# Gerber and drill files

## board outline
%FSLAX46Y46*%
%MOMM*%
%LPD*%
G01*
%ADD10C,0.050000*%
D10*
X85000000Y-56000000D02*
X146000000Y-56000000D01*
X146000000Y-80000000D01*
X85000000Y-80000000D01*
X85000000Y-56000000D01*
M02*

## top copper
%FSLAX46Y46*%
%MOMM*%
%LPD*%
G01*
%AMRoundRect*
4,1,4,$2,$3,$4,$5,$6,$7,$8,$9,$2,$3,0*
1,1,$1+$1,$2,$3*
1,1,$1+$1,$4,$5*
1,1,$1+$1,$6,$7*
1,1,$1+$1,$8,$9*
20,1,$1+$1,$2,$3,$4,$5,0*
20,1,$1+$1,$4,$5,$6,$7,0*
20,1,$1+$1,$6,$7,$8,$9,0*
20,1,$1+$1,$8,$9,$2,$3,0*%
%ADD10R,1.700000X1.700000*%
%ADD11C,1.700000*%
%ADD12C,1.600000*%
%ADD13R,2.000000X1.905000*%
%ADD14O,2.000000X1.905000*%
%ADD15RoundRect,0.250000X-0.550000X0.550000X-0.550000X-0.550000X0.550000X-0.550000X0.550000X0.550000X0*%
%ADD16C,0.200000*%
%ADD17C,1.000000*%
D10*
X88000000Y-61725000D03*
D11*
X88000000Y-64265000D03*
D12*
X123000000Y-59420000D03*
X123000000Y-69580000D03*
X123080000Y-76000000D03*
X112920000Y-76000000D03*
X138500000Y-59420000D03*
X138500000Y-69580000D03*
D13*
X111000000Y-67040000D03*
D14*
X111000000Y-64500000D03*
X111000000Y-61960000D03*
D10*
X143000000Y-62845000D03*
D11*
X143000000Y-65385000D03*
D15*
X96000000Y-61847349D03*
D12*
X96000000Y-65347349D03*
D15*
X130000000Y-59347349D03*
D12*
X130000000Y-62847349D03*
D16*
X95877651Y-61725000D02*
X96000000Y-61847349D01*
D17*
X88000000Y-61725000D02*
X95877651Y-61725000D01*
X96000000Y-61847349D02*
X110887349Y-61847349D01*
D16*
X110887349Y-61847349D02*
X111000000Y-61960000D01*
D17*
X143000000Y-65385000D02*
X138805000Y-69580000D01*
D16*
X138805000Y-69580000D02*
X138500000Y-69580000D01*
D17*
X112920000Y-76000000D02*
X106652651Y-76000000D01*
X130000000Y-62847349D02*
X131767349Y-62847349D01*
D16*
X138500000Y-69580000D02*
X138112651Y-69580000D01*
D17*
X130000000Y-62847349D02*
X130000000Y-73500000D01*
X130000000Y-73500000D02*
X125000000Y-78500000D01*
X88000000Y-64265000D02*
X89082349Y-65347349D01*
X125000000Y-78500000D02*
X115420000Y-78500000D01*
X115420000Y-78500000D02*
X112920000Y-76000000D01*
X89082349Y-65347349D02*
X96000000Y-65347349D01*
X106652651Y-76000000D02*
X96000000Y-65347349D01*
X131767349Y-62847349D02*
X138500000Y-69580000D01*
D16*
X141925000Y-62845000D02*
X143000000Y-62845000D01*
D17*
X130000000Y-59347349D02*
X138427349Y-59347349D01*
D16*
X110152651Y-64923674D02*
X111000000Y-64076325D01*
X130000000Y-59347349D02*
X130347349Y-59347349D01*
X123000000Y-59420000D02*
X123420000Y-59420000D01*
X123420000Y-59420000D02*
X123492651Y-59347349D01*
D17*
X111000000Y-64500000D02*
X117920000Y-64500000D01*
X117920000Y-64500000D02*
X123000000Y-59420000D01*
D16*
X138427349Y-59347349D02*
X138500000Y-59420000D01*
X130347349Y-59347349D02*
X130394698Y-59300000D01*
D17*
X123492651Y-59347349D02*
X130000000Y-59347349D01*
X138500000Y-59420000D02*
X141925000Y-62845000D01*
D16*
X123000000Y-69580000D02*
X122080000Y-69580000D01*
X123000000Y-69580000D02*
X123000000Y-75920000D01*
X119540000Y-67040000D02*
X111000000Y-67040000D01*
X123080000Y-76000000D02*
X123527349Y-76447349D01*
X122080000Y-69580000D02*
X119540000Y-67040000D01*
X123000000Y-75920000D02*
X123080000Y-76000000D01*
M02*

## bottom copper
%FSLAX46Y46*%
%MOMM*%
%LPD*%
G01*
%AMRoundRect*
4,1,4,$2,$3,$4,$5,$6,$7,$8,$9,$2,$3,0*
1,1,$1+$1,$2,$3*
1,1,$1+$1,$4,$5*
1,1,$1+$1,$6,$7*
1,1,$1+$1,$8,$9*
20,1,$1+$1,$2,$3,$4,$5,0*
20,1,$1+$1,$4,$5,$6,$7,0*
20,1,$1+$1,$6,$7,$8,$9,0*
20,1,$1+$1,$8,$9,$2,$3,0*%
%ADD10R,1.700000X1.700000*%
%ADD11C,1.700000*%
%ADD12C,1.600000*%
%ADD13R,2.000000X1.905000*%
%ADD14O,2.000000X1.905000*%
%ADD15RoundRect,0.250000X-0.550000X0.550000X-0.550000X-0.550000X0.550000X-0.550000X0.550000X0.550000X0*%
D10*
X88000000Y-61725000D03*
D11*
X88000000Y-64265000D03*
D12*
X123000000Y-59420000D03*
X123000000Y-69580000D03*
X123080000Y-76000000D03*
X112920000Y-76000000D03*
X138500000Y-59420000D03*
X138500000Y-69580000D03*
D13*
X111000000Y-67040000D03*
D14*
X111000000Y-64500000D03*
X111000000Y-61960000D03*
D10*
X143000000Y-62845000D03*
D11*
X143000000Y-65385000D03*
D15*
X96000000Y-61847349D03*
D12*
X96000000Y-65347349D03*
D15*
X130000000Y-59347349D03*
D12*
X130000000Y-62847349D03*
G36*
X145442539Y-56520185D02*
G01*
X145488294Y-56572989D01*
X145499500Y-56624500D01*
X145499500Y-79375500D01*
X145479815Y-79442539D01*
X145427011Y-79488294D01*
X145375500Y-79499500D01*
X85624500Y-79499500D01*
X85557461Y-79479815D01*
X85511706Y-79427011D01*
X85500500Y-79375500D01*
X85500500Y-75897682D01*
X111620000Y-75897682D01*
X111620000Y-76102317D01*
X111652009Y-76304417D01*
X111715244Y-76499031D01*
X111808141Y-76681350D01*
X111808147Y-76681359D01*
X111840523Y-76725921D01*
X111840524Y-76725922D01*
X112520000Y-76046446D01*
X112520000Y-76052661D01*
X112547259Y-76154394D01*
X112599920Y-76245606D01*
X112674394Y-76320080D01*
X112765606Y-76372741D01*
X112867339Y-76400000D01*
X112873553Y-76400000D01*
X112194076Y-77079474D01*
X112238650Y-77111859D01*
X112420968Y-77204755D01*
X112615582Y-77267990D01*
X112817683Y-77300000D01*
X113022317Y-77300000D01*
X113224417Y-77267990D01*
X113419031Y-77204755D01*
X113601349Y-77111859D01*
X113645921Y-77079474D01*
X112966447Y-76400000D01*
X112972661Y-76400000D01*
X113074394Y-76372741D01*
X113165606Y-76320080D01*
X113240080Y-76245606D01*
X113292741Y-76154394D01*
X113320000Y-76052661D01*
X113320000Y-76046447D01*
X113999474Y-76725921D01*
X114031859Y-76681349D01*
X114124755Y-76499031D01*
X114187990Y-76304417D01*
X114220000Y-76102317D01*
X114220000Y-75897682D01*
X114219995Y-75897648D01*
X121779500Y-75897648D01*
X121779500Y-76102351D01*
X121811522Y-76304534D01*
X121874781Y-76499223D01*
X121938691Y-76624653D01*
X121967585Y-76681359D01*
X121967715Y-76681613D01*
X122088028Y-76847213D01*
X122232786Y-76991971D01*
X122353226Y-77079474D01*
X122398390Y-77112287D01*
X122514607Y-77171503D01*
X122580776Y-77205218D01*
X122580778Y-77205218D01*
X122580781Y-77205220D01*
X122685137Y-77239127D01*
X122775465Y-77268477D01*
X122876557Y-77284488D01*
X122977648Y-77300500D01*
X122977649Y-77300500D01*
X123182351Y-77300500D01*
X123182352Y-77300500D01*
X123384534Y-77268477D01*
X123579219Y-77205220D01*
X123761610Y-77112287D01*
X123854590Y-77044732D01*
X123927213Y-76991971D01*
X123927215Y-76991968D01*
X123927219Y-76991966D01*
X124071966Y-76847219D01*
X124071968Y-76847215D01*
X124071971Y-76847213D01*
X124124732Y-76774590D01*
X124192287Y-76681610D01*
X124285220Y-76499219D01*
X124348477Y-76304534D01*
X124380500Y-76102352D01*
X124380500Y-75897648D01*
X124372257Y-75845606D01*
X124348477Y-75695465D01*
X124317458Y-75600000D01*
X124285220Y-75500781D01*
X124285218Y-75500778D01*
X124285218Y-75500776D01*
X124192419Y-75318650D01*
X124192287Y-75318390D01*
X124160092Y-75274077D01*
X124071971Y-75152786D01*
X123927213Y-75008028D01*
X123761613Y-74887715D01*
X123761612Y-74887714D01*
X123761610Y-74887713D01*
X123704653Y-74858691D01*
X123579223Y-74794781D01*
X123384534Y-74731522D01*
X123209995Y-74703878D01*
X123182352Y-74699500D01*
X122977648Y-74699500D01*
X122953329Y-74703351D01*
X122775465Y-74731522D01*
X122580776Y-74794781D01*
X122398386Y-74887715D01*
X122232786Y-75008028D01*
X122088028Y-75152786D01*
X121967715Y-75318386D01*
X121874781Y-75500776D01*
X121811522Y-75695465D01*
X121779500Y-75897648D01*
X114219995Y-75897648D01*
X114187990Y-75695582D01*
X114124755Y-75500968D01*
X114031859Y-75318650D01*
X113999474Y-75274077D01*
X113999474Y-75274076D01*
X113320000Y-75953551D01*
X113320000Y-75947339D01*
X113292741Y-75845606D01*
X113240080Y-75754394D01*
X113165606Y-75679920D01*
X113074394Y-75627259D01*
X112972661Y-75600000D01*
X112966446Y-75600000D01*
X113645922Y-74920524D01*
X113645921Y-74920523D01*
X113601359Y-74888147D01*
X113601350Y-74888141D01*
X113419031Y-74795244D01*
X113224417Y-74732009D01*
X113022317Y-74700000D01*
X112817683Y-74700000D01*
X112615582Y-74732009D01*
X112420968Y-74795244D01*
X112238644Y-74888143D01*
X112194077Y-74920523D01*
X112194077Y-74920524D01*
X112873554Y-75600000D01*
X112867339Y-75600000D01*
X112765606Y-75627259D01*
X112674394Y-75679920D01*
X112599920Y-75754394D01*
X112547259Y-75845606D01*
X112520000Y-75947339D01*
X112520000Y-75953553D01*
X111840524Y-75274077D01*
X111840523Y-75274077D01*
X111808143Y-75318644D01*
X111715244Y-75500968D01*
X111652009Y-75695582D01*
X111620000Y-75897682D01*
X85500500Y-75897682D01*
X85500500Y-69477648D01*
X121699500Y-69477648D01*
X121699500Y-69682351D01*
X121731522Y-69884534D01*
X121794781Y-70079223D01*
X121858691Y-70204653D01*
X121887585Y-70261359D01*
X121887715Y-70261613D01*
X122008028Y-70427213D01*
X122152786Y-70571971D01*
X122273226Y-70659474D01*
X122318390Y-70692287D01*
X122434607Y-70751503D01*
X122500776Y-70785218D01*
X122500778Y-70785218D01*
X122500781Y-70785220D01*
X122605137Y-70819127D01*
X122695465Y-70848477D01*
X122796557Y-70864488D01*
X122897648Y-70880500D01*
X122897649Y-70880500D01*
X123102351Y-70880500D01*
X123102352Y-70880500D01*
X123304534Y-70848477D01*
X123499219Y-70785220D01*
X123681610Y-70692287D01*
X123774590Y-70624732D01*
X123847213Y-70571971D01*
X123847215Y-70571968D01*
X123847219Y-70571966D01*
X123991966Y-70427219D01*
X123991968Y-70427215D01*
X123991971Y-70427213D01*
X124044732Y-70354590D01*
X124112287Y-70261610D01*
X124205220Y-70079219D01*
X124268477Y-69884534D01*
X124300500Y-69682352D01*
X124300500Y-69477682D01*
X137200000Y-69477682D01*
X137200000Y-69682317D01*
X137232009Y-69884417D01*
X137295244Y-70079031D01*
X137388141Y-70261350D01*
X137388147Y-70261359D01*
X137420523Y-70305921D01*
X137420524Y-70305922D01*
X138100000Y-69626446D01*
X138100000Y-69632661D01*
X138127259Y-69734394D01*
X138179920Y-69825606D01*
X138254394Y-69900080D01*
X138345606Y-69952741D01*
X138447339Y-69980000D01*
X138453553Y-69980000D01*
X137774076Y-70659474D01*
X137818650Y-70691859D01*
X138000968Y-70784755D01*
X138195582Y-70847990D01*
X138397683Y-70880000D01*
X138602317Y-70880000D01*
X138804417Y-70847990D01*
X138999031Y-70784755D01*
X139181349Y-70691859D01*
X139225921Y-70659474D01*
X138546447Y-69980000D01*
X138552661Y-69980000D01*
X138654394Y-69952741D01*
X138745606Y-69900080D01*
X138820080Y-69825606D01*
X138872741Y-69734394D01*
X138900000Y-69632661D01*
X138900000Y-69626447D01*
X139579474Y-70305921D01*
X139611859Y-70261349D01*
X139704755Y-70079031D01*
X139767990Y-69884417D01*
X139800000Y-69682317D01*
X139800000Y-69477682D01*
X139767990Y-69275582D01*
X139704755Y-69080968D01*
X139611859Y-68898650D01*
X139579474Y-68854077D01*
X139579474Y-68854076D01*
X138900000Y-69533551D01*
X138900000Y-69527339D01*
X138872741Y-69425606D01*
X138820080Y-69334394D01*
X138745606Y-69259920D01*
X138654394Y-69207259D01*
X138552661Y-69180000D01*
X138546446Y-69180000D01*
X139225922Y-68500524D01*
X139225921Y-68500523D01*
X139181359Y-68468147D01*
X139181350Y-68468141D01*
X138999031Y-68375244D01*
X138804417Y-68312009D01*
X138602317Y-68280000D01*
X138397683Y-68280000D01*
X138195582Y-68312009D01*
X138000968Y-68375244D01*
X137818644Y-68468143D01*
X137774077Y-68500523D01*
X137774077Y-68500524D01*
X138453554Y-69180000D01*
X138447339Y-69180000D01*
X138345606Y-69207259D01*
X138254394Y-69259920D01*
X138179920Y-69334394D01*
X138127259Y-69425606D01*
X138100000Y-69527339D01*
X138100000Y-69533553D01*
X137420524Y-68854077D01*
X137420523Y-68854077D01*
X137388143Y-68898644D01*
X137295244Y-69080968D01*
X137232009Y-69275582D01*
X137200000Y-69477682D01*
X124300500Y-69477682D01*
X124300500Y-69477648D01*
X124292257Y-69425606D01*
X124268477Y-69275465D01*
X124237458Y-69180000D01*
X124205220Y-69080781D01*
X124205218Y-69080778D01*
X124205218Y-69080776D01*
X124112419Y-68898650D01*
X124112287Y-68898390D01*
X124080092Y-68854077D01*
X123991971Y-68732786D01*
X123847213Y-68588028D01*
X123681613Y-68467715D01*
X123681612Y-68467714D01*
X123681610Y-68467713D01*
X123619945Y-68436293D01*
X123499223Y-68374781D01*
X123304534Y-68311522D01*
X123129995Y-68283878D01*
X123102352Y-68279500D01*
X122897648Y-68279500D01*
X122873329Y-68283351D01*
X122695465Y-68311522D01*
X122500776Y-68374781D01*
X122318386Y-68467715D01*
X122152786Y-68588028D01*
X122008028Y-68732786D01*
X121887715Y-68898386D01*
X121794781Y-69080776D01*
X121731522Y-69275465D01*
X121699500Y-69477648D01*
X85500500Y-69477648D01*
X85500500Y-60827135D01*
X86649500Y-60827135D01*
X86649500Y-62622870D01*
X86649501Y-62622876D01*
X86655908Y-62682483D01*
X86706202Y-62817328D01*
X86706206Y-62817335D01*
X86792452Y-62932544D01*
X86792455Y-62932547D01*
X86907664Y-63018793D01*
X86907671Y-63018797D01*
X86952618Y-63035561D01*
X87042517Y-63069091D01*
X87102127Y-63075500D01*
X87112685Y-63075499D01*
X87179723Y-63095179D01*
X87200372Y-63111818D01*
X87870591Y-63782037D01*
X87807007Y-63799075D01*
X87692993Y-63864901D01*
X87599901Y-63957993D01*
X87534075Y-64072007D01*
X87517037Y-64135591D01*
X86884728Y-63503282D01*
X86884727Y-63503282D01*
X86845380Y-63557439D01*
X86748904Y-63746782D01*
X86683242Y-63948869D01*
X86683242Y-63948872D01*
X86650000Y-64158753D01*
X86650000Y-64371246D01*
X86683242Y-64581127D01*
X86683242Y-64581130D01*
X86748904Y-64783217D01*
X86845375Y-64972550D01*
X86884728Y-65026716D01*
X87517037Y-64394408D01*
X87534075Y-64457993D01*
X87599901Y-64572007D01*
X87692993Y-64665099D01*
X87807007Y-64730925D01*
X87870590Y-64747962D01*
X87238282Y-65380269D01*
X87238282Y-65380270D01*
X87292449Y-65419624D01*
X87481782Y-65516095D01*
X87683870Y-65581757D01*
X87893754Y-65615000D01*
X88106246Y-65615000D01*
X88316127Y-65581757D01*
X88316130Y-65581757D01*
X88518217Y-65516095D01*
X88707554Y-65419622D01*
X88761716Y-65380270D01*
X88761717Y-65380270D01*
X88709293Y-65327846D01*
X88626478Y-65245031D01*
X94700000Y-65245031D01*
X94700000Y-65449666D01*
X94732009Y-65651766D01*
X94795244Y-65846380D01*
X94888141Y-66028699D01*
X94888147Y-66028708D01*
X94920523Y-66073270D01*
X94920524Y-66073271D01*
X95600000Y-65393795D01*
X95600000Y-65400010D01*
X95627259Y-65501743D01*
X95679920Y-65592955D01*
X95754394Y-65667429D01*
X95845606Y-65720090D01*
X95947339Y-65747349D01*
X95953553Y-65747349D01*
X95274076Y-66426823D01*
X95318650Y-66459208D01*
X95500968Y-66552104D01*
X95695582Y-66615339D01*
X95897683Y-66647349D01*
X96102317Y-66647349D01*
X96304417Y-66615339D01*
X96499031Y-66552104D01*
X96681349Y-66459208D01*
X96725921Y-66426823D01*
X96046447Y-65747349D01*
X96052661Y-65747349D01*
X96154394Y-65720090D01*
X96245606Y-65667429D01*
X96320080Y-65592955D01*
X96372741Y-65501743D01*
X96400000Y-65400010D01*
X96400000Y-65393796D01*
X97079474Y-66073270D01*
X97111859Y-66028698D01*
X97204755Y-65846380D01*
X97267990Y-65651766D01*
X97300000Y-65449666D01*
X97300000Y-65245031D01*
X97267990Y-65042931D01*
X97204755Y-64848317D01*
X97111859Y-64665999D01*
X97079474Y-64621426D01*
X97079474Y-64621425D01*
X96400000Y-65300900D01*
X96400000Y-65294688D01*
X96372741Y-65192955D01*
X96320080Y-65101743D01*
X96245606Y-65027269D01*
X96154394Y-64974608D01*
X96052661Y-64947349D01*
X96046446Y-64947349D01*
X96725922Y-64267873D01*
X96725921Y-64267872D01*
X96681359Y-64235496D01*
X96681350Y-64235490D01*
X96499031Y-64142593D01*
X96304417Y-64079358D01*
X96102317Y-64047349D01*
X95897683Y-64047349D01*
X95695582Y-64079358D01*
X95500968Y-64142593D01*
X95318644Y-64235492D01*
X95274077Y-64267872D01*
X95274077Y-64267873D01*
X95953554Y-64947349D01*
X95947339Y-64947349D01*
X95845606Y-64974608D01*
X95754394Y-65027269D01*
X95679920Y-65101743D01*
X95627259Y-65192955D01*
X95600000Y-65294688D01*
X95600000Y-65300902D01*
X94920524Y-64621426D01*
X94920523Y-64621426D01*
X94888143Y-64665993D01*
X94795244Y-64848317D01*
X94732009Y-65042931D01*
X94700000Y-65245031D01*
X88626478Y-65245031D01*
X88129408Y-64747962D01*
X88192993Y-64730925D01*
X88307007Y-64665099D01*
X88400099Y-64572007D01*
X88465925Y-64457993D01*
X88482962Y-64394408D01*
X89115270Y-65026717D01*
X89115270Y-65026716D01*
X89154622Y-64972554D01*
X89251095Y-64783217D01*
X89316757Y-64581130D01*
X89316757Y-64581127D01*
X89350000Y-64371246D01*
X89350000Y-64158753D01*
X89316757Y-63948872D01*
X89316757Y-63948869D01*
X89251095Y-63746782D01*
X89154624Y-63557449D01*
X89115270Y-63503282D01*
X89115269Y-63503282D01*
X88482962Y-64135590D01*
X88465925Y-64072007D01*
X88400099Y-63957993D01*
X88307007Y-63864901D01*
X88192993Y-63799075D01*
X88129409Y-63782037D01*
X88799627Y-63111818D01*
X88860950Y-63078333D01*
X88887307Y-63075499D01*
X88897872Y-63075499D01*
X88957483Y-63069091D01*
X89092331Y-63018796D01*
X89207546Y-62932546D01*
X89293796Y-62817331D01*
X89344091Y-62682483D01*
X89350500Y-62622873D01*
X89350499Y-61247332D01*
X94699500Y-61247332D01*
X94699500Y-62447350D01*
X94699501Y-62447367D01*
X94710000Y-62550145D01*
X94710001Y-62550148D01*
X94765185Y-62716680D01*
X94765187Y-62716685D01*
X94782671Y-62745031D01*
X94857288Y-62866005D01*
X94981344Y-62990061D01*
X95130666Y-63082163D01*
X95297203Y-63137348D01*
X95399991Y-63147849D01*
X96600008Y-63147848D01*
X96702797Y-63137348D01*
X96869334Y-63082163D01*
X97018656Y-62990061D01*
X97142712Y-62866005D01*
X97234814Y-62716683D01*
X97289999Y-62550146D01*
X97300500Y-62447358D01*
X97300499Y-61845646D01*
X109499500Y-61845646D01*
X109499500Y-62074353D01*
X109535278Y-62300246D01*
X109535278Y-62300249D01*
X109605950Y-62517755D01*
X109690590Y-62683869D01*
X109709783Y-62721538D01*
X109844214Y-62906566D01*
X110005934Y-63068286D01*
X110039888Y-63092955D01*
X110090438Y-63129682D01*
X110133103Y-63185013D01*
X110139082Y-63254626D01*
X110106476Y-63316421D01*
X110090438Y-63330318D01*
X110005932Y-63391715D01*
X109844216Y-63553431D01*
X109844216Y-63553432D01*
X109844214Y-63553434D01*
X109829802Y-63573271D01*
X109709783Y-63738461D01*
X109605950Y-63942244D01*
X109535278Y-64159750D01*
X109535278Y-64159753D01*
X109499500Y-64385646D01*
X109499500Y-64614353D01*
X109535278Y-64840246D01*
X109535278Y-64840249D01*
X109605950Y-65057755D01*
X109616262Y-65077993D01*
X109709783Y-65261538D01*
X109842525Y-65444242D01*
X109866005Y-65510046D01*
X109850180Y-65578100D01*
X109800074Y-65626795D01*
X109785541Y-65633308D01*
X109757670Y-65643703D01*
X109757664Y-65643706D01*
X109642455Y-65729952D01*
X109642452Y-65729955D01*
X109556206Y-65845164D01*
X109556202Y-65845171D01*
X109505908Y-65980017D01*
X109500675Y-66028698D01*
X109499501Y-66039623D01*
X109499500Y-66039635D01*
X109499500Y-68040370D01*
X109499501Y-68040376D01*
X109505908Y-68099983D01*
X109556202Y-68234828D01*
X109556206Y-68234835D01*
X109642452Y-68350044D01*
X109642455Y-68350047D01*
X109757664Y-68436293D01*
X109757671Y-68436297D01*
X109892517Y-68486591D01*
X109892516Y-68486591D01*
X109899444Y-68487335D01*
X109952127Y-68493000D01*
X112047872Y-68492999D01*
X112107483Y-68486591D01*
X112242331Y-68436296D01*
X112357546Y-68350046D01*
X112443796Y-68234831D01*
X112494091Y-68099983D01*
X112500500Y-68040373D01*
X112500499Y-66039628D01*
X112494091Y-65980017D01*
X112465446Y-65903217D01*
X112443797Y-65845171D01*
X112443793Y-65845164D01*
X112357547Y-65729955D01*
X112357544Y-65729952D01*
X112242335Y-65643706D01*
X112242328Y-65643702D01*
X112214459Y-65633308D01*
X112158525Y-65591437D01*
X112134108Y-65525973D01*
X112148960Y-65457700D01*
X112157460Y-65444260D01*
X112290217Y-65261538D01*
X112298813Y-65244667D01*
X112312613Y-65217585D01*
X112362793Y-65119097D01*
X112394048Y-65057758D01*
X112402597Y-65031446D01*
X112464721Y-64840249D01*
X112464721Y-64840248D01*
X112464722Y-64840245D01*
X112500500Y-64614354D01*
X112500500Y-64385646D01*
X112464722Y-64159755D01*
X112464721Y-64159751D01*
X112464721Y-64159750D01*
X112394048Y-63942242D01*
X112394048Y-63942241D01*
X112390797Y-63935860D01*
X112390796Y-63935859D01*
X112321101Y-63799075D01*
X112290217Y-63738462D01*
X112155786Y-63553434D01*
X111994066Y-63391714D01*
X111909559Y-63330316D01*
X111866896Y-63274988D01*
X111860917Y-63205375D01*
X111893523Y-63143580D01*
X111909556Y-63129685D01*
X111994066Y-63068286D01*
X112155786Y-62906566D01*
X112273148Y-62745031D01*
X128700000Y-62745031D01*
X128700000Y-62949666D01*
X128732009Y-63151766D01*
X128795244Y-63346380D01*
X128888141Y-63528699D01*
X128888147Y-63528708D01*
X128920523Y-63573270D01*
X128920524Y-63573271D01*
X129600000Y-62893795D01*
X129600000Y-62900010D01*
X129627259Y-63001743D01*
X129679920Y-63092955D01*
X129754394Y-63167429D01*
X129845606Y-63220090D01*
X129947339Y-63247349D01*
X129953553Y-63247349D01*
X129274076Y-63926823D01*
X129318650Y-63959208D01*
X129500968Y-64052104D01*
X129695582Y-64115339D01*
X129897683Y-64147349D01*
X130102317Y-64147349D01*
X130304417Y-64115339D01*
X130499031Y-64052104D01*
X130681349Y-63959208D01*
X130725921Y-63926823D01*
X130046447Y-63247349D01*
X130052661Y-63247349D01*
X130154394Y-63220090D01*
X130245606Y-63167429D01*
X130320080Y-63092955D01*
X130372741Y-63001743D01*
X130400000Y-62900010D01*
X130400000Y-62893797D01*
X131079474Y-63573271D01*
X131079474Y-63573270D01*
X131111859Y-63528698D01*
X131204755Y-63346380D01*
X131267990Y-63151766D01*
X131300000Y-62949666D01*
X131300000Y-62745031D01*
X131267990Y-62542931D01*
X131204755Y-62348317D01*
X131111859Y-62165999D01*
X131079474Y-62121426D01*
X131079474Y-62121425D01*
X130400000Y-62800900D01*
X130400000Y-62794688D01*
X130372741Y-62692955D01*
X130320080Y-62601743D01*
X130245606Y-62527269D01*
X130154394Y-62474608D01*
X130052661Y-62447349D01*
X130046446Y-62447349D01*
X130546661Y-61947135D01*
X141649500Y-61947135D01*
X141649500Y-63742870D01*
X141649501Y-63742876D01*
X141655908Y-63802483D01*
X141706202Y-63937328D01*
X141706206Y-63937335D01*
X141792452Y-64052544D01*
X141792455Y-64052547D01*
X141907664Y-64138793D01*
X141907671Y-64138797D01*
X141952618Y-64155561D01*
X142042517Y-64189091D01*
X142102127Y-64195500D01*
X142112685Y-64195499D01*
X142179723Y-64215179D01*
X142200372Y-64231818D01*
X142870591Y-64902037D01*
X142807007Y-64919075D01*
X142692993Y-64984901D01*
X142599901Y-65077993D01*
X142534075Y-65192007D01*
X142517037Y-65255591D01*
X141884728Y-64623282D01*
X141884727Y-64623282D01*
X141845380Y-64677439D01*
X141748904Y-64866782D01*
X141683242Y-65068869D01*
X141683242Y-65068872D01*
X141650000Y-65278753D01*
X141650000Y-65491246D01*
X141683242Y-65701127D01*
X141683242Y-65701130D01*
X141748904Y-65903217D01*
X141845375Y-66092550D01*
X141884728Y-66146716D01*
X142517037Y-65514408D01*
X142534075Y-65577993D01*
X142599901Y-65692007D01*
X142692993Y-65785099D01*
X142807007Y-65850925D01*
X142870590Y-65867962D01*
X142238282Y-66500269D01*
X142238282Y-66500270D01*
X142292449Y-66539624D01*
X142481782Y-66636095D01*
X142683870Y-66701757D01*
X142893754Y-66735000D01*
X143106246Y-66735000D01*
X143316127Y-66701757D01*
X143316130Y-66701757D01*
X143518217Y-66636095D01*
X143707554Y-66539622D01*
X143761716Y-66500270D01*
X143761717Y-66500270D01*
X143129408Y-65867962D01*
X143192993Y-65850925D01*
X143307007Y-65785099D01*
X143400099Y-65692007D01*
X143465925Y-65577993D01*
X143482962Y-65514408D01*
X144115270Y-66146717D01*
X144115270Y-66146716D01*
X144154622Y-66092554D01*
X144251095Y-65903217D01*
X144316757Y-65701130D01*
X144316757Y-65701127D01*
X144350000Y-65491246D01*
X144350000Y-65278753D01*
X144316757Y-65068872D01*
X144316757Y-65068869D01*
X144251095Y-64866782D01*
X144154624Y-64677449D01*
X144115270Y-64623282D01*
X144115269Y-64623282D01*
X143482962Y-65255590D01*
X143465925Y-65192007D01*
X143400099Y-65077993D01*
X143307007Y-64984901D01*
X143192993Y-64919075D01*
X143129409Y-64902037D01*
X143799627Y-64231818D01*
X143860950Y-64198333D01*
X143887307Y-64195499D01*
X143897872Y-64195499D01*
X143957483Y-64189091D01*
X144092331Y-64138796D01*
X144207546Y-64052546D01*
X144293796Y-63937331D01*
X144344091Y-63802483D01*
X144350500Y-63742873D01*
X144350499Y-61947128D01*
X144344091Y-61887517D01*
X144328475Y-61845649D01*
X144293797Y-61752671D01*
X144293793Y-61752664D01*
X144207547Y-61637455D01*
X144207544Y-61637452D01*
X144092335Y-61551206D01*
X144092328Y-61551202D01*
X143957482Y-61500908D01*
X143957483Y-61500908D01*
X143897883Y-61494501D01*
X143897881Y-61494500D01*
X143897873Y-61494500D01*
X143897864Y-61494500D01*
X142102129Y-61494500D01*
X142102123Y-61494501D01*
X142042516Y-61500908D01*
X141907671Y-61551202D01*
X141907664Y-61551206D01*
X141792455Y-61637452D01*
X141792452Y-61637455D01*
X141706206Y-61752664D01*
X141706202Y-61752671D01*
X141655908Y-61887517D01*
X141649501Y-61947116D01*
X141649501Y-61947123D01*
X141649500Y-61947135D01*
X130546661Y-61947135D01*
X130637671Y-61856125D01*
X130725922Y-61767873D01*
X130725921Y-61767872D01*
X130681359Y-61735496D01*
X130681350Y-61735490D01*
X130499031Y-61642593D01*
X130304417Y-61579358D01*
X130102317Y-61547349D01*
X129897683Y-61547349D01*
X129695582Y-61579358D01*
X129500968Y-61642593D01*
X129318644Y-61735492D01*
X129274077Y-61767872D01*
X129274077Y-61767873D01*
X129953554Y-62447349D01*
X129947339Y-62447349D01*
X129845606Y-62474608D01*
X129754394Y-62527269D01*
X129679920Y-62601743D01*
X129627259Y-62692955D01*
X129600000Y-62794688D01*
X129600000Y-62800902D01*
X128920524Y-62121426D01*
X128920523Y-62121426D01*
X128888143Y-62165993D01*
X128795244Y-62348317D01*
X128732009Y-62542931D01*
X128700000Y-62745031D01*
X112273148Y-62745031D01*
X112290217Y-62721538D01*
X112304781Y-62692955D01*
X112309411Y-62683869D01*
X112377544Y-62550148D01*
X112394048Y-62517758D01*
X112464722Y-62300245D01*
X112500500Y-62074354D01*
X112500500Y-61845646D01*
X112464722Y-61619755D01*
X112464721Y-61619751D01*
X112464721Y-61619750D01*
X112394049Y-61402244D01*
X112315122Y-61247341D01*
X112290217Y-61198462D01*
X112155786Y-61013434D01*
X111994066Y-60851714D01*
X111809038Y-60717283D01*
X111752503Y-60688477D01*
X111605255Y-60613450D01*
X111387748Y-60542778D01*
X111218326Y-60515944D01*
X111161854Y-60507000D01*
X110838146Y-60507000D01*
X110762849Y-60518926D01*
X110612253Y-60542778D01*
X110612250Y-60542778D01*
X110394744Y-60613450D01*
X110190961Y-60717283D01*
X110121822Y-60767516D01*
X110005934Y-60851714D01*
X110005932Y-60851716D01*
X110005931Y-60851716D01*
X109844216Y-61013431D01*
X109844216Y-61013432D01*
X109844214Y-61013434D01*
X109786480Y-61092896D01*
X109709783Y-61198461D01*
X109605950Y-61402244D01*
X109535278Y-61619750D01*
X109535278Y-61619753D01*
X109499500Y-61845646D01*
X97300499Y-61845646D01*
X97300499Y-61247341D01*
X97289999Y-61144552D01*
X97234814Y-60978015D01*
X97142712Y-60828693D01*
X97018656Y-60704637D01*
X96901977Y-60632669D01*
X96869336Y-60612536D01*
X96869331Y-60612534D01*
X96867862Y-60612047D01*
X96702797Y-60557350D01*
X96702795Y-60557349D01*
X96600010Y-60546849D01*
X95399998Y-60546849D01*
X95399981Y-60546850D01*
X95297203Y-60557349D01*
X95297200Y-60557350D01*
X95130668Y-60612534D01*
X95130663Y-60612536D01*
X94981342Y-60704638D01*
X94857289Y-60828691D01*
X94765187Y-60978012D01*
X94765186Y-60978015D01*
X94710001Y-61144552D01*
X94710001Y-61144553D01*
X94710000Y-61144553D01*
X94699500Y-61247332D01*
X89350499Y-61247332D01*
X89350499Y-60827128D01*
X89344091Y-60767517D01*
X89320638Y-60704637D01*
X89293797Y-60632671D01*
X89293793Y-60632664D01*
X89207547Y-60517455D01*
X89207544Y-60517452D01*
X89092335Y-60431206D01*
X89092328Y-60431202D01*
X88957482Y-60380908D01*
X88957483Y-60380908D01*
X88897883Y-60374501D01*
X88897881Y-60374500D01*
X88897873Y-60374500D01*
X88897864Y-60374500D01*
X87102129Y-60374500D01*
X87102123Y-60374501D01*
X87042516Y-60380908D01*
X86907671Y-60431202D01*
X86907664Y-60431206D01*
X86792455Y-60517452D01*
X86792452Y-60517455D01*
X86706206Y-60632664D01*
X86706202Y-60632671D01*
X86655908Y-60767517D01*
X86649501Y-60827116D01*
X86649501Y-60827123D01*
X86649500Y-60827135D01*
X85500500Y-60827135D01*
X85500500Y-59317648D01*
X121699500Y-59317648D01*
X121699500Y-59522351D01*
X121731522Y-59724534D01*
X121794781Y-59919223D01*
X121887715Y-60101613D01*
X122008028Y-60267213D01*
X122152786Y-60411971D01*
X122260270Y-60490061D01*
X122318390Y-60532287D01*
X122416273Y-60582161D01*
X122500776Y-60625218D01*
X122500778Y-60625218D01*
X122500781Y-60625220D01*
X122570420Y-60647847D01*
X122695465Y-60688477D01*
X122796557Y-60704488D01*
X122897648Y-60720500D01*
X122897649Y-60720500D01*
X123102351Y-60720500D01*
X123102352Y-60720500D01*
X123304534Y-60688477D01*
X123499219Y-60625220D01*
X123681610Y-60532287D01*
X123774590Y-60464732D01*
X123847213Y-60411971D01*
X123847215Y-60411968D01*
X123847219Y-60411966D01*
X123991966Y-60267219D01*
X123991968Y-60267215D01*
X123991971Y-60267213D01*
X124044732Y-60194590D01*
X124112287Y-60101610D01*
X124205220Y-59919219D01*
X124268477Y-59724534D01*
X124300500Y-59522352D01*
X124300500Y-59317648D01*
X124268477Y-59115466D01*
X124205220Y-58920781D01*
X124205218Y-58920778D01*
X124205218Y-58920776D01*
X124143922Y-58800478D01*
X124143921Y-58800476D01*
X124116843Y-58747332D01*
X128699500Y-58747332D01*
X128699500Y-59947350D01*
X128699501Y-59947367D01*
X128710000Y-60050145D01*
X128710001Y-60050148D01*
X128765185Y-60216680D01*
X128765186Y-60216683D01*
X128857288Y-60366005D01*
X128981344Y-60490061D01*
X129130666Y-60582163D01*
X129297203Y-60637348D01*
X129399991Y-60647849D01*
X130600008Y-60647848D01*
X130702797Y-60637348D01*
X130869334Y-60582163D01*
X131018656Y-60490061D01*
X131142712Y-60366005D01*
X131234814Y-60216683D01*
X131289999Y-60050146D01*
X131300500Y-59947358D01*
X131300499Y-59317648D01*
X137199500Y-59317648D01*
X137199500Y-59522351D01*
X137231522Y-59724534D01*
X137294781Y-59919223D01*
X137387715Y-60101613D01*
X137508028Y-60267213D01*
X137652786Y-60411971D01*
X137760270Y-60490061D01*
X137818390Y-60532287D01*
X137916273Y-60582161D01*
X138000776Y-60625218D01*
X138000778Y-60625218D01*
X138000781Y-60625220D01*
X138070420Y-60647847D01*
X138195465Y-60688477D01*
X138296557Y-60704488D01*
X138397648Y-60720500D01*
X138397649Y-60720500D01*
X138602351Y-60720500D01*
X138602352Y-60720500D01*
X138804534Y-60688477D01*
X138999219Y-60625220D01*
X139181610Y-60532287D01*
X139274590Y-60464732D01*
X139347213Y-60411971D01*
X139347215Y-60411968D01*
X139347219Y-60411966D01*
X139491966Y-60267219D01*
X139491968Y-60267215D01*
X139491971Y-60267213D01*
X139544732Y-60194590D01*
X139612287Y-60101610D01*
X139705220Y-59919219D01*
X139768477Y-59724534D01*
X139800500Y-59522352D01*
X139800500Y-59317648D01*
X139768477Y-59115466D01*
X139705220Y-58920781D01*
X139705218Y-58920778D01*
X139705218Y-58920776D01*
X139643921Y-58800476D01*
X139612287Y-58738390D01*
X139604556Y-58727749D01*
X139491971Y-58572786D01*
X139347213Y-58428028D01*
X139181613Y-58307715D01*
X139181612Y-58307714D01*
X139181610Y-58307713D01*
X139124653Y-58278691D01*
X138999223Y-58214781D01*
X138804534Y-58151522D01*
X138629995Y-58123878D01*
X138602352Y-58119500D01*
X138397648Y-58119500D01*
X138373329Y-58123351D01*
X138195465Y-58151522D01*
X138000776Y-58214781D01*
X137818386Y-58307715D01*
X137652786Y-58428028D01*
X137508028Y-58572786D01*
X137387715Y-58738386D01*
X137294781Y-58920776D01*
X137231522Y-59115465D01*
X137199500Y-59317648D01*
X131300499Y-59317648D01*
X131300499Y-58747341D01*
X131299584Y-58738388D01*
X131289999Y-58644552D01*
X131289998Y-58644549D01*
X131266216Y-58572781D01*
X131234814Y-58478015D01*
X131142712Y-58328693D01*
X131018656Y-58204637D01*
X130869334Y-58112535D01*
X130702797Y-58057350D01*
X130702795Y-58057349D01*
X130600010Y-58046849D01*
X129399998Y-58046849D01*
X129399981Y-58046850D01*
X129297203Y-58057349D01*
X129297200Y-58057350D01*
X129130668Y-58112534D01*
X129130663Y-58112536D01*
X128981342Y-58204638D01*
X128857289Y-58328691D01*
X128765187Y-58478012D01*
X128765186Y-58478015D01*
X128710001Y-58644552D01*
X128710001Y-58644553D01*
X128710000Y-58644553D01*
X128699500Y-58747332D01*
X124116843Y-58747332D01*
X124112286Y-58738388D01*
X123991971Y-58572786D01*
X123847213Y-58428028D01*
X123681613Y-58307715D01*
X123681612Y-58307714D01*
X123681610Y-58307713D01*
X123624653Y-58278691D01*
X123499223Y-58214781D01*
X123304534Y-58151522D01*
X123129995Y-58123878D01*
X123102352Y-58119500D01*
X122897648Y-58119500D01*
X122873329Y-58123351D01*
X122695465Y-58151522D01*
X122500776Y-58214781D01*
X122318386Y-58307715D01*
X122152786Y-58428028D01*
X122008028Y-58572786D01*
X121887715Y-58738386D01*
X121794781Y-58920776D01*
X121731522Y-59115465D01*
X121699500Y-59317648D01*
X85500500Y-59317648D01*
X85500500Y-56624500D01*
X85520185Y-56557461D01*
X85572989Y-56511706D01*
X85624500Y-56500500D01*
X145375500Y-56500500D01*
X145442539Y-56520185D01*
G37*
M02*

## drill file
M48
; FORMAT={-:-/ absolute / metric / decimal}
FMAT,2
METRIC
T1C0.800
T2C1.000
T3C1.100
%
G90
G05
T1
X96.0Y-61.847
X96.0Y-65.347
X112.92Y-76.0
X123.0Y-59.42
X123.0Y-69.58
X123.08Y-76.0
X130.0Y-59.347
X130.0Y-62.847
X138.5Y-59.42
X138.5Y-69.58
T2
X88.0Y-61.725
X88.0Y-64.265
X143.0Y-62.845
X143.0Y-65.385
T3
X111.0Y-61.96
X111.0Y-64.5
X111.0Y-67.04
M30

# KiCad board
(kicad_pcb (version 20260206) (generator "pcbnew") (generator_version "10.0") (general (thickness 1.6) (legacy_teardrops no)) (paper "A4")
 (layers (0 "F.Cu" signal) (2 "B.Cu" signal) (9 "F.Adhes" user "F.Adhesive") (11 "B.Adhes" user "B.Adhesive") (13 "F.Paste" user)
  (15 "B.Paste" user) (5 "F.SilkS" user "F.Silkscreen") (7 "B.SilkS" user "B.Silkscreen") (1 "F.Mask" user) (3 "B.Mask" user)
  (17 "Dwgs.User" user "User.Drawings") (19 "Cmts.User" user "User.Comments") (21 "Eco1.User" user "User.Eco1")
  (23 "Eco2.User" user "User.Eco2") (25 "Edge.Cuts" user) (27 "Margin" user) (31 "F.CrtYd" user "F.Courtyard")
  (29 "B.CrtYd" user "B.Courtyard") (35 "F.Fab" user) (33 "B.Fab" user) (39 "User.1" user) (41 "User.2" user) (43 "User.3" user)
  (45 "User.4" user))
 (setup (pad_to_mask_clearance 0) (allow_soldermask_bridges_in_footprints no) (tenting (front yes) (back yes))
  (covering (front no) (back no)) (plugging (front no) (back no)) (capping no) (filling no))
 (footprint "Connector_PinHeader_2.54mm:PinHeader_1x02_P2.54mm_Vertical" (layer "F.Cu") (at 88 61.725)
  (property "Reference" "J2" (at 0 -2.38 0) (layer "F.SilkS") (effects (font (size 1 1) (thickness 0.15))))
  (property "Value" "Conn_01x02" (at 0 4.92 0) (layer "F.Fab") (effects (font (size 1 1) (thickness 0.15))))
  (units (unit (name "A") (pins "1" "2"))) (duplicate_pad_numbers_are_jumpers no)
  (pad "1" thru_hole rect (at 0 0) (size 1.7 1.7) (drill 1) (layers "*.Cu" "*.Mask") (remove_unused_layers no) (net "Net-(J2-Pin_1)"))
  (pad "2" thru_hole circle (at 0 2.54) (size 1.7 1.7) (drill 1) (layers "*.Cu" "*.Mask") (remove_unused_layers no) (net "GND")))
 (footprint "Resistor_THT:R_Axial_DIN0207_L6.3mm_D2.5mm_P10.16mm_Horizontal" (layer "F.Cu") (at 123 59.42 -90)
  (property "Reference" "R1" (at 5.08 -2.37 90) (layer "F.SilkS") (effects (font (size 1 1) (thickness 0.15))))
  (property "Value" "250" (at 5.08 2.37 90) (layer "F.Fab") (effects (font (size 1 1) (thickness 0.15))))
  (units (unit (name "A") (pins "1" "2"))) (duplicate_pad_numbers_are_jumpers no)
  (pad "1" thru_hole circle (at 0 0 270) (size 1.6 1.6) (drill 0.8) (layers "*.Cu" "*.Mask") (remove_unused_layers no)
   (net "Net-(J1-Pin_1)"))
  (pad "2" thru_hole circle (at 10.16 0 270) (size 1.6 1.6) (drill 0.8) (layers "*.Cu" "*.Mask") (remove_unused_layers no)
   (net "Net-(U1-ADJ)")))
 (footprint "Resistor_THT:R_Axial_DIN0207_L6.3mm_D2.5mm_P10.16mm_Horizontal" (layer "F.Cu") (at 123.08 76 180)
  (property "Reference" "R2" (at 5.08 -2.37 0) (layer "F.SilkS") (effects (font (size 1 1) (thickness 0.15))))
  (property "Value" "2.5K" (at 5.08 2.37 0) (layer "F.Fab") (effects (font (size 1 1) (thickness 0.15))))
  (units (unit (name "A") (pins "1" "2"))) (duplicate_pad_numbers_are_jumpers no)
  (pad "1" thru_hole circle (at 0 0 180) (size 1.6 1.6) (drill 0.8) (layers "*.Cu" "*.Mask") (remove_unused_layers no) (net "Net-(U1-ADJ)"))
  (pad "2" thru_hole circle (at 10.16 0 180) (size 1.6 1.6) (drill 0.8) (layers "*.Cu" "*.Mask") (remove_unused_layers no) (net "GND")))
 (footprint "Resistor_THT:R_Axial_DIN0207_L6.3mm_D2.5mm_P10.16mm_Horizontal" (layer "F.Cu") (at 138.5 59.42 -90)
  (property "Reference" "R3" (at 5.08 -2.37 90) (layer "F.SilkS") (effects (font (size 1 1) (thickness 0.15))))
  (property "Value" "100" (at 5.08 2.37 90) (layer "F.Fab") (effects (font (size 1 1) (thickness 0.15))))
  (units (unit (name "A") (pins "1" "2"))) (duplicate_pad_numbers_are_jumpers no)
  (pad "1" thru_hole circle (at 0 0 270) (size 1.6 1.6) (drill 0.8) (layers "*.Cu" "*.Mask") (remove_unused_layers no)
   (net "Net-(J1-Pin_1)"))
  (pad "2" thru_hole circle (at 10.16 0 270) (size 1.6 1.6) (drill 0.8) (layers "*.Cu" "*.Mask") (remove_unused_layers no) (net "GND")))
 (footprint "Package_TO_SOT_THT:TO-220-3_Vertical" (layer "F.Cu") (at 111 67.04 90)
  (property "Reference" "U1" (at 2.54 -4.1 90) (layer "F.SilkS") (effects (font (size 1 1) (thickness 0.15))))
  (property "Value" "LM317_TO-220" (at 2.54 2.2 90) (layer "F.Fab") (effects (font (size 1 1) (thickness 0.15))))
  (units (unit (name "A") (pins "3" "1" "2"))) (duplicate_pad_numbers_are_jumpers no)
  (pad "1" thru_hole rect (at 0 0 90) (size 1.905 2) (drill 1.1) (layers "*.Cu" "*.Mask") (remove_unused_layers no) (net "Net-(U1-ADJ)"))
  (pad "2" thru_hole oval (at 2.54 0 90) (size 1.905 2) (drill 1.1) (layers "*.Cu" "*.Mask") (remove_unused_layers no)
   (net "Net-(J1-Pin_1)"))
  (pad "3" thru_hole oval (at 5.08 0 90) (size 1.905 2) (drill 1.1) (layers "*.Cu" "*.Mask") (remove_unused_layers no)
   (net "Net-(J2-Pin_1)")))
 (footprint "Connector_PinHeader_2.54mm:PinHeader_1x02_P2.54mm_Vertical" (layer "F.Cu") (at 143 62.845)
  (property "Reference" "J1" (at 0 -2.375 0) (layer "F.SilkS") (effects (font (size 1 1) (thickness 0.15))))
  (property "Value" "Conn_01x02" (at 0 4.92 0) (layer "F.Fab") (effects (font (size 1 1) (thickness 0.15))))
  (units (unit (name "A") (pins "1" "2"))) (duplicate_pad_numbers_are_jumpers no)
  (pad "1" thru_hole rect (at 0 0) (size 1.7 1.7) (drill 1) (layers "*.Cu" "*.Mask") (remove_unused_layers no) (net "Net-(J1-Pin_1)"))
  (pad "2" thru_hole circle (at 0 2.54) (size 1.7 1.7) (drill 1) (layers "*.Cu" "*.Mask") (remove_unused_layers no) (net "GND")))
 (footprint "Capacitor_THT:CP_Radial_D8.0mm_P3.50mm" (layer "F.Cu") (at 96 61.847349 -90)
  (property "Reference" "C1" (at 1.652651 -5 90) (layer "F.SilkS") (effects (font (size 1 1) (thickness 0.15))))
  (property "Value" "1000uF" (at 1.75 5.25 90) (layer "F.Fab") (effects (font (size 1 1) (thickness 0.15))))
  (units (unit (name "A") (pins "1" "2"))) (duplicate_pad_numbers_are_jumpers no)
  (pad "1" thru_hole roundrect (at 0 0 270) (size 1.6 1.6) (drill 0.8) (layers "*.Cu" "*.Mask") (remove_unused_layers no)
   (roundrect_rratio 0.15625) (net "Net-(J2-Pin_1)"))
  (pad "2" thru_hole circle (at 3.5 0 270) (size 1.6 1.6) (drill 0.8) (layers "*.Cu" "*.Mask") (remove_unused_layers no) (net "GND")))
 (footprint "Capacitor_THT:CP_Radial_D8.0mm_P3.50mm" (layer "F.Cu") (at 130 59.347349 -90)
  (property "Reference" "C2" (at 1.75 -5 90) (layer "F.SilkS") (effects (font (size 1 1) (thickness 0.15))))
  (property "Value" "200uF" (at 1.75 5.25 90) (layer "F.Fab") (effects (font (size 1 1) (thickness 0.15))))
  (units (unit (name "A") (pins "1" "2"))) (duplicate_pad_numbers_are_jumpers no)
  (pad "1" thru_hole roundrect (at 0 0 270) (size 1.6 1.6) (drill 0.8) (layers "*.Cu" "*.Mask") (remove_unused_layers no)
   (roundrect_rratio 0.15625) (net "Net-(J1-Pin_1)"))
  (pad "2" thru_hole circle (at 3.5 0 270) (size 1.6 1.6) (drill 0.8) (layers "*.Cu" "*.Mask") (remove_unused_layers no) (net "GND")))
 (gr_rect (start 85 56) (end 146 80) (stroke (width 0.05) (type default)) (fill no) (layer "Edge.Cuts"))
 (segment (start 95.877651 61.725) (end 96 61.847349) (width 0.2) (layer "F.Cu") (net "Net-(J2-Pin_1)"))
 (segment (start 88 61.725) (end 95.877651 61.725) (width 1) (layer "F.Cu") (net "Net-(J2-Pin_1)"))
 (segment (start 96 61.847349) (end 110.887349 61.847349) (width 1) (layer "F.Cu") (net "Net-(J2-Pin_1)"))
 (segment (start 110.887349 61.847349) (end 111 61.96) (width 0.2) (layer "F.Cu") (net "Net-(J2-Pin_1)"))
 (segment (start 143 65.385) (end 138.805 69.58) (width 1) (layer "F.Cu") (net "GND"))
 (segment (start 138.805 69.58) (end 138.5 69.58) (width 0.2) (layer "F.Cu") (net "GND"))
 (segment (start 112.92 76) (end 106.652651 76) (width 1) (layer "F.Cu") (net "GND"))
 (segment (start 130 62.847349) (end 131.767349 62.847349) (width 1) (layer "F.Cu") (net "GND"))
 (segment (start 138.5 69.58) (end 138.112651 69.58) (width 0.2) (layer "F.Cu") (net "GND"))
 (segment (start 130 62.847349) (end 130 73.5) (width 1) (layer "F.Cu") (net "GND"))
 (segment (start 130 73.5) (end 125 78.5) (width 1) (layer "F.Cu") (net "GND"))
 (segment (start 88 64.265) (end 89.082349 65.347349) (width 1) (layer "F.Cu") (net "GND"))
 (segment (start 125 78.5) (end 115.42 78.5) (width 1) (layer "F.Cu") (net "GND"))
 (segment (start 115.42 78.5) (end 112.92 76) (width 1) (layer "F.Cu") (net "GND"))
 (segment (start 89.082349 65.347349) (end 96 65.347349) (width 1) (layer "F.Cu") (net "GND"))
 (segment (start 106.652651 76) (end 96 65.347349) (width 1) (layer "F.Cu") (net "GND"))
 (segment (start 131.767349 62.847349) (end 138.5 69.58) (width 1) (layer "F.Cu") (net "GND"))
 (segment (start 141.925 62.845) (end 143 62.845) (width 0.2) (layer "F.Cu") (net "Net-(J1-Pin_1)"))
 (segment (start 130 59.347349) (end 138.427349 59.347349) (width 1) (layer "F.Cu") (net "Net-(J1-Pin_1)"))
 (segment (start 110.152651 64.923674) (end 111 64.076325) (width 0.2) (layer "F.Cu") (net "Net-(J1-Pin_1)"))
 (segment (start 130 59.347349) (end 130.347349 59.347349) (width 0.2) (layer "F.Cu") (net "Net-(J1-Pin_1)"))
 (segment (start 123 59.42) (end 123.42 59.42) (width 0.2) (layer "F.Cu") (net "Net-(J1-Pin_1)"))
 (segment (start 123.42 59.42) (end 123.492651 59.347349) (width 0.2) (layer "F.Cu") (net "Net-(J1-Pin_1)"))
 (segment (start 111 64.5) (end 117.92 64.5) (width 1) (layer "F.Cu") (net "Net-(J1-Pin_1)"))
 (segment (start 117.92 64.5) (end 123 59.42) (width 1) (layer "F.Cu") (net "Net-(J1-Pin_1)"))
 (segment (start 138.427349 59.347349) (end 138.5 59.42) (width 0.2) (layer "F.Cu") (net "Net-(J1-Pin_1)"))
 (segment (start 130.347349 59.347349) (end 130.394698 59.3) (width 0.2) (layer "F.Cu") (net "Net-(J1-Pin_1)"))
 (segment (start 123.492651 59.347349) (end 130 59.347349) (width 1) (layer "F.Cu") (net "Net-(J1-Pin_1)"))
 (segment (start 138.5 59.42) (end 141.925 62.845) (width 1) (layer "F.Cu") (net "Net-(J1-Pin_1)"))
 (segment (start 123 69.58) (end 122.08 69.58) (width 0.2) (layer "F.Cu") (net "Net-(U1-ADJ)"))
 (segment (start 123 69.58) (end 123 75.92) (width 0.2) (layer "F.Cu") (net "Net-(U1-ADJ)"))
 (segment (start 119.54 67.04) (end 111 67.04) (width 0.2) (layer "F.Cu") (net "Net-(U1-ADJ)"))
 (segment (start 123.08 76) (end 123.527349 76.447349) (width 0.2) (layer "F.Cu") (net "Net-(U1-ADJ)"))
 (segment (start 122.08 69.58) (end 119.54 67.04) (width 0.2) (layer "F.Cu") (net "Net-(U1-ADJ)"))
 (segment (start 123 75.92) (end 123.08 76) (width 0.2) (layer "F.Cu") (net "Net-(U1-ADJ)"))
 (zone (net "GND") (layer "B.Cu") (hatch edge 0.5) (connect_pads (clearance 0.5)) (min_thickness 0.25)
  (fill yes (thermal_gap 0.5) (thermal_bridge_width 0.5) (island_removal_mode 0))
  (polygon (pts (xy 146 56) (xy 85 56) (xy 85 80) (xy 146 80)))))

